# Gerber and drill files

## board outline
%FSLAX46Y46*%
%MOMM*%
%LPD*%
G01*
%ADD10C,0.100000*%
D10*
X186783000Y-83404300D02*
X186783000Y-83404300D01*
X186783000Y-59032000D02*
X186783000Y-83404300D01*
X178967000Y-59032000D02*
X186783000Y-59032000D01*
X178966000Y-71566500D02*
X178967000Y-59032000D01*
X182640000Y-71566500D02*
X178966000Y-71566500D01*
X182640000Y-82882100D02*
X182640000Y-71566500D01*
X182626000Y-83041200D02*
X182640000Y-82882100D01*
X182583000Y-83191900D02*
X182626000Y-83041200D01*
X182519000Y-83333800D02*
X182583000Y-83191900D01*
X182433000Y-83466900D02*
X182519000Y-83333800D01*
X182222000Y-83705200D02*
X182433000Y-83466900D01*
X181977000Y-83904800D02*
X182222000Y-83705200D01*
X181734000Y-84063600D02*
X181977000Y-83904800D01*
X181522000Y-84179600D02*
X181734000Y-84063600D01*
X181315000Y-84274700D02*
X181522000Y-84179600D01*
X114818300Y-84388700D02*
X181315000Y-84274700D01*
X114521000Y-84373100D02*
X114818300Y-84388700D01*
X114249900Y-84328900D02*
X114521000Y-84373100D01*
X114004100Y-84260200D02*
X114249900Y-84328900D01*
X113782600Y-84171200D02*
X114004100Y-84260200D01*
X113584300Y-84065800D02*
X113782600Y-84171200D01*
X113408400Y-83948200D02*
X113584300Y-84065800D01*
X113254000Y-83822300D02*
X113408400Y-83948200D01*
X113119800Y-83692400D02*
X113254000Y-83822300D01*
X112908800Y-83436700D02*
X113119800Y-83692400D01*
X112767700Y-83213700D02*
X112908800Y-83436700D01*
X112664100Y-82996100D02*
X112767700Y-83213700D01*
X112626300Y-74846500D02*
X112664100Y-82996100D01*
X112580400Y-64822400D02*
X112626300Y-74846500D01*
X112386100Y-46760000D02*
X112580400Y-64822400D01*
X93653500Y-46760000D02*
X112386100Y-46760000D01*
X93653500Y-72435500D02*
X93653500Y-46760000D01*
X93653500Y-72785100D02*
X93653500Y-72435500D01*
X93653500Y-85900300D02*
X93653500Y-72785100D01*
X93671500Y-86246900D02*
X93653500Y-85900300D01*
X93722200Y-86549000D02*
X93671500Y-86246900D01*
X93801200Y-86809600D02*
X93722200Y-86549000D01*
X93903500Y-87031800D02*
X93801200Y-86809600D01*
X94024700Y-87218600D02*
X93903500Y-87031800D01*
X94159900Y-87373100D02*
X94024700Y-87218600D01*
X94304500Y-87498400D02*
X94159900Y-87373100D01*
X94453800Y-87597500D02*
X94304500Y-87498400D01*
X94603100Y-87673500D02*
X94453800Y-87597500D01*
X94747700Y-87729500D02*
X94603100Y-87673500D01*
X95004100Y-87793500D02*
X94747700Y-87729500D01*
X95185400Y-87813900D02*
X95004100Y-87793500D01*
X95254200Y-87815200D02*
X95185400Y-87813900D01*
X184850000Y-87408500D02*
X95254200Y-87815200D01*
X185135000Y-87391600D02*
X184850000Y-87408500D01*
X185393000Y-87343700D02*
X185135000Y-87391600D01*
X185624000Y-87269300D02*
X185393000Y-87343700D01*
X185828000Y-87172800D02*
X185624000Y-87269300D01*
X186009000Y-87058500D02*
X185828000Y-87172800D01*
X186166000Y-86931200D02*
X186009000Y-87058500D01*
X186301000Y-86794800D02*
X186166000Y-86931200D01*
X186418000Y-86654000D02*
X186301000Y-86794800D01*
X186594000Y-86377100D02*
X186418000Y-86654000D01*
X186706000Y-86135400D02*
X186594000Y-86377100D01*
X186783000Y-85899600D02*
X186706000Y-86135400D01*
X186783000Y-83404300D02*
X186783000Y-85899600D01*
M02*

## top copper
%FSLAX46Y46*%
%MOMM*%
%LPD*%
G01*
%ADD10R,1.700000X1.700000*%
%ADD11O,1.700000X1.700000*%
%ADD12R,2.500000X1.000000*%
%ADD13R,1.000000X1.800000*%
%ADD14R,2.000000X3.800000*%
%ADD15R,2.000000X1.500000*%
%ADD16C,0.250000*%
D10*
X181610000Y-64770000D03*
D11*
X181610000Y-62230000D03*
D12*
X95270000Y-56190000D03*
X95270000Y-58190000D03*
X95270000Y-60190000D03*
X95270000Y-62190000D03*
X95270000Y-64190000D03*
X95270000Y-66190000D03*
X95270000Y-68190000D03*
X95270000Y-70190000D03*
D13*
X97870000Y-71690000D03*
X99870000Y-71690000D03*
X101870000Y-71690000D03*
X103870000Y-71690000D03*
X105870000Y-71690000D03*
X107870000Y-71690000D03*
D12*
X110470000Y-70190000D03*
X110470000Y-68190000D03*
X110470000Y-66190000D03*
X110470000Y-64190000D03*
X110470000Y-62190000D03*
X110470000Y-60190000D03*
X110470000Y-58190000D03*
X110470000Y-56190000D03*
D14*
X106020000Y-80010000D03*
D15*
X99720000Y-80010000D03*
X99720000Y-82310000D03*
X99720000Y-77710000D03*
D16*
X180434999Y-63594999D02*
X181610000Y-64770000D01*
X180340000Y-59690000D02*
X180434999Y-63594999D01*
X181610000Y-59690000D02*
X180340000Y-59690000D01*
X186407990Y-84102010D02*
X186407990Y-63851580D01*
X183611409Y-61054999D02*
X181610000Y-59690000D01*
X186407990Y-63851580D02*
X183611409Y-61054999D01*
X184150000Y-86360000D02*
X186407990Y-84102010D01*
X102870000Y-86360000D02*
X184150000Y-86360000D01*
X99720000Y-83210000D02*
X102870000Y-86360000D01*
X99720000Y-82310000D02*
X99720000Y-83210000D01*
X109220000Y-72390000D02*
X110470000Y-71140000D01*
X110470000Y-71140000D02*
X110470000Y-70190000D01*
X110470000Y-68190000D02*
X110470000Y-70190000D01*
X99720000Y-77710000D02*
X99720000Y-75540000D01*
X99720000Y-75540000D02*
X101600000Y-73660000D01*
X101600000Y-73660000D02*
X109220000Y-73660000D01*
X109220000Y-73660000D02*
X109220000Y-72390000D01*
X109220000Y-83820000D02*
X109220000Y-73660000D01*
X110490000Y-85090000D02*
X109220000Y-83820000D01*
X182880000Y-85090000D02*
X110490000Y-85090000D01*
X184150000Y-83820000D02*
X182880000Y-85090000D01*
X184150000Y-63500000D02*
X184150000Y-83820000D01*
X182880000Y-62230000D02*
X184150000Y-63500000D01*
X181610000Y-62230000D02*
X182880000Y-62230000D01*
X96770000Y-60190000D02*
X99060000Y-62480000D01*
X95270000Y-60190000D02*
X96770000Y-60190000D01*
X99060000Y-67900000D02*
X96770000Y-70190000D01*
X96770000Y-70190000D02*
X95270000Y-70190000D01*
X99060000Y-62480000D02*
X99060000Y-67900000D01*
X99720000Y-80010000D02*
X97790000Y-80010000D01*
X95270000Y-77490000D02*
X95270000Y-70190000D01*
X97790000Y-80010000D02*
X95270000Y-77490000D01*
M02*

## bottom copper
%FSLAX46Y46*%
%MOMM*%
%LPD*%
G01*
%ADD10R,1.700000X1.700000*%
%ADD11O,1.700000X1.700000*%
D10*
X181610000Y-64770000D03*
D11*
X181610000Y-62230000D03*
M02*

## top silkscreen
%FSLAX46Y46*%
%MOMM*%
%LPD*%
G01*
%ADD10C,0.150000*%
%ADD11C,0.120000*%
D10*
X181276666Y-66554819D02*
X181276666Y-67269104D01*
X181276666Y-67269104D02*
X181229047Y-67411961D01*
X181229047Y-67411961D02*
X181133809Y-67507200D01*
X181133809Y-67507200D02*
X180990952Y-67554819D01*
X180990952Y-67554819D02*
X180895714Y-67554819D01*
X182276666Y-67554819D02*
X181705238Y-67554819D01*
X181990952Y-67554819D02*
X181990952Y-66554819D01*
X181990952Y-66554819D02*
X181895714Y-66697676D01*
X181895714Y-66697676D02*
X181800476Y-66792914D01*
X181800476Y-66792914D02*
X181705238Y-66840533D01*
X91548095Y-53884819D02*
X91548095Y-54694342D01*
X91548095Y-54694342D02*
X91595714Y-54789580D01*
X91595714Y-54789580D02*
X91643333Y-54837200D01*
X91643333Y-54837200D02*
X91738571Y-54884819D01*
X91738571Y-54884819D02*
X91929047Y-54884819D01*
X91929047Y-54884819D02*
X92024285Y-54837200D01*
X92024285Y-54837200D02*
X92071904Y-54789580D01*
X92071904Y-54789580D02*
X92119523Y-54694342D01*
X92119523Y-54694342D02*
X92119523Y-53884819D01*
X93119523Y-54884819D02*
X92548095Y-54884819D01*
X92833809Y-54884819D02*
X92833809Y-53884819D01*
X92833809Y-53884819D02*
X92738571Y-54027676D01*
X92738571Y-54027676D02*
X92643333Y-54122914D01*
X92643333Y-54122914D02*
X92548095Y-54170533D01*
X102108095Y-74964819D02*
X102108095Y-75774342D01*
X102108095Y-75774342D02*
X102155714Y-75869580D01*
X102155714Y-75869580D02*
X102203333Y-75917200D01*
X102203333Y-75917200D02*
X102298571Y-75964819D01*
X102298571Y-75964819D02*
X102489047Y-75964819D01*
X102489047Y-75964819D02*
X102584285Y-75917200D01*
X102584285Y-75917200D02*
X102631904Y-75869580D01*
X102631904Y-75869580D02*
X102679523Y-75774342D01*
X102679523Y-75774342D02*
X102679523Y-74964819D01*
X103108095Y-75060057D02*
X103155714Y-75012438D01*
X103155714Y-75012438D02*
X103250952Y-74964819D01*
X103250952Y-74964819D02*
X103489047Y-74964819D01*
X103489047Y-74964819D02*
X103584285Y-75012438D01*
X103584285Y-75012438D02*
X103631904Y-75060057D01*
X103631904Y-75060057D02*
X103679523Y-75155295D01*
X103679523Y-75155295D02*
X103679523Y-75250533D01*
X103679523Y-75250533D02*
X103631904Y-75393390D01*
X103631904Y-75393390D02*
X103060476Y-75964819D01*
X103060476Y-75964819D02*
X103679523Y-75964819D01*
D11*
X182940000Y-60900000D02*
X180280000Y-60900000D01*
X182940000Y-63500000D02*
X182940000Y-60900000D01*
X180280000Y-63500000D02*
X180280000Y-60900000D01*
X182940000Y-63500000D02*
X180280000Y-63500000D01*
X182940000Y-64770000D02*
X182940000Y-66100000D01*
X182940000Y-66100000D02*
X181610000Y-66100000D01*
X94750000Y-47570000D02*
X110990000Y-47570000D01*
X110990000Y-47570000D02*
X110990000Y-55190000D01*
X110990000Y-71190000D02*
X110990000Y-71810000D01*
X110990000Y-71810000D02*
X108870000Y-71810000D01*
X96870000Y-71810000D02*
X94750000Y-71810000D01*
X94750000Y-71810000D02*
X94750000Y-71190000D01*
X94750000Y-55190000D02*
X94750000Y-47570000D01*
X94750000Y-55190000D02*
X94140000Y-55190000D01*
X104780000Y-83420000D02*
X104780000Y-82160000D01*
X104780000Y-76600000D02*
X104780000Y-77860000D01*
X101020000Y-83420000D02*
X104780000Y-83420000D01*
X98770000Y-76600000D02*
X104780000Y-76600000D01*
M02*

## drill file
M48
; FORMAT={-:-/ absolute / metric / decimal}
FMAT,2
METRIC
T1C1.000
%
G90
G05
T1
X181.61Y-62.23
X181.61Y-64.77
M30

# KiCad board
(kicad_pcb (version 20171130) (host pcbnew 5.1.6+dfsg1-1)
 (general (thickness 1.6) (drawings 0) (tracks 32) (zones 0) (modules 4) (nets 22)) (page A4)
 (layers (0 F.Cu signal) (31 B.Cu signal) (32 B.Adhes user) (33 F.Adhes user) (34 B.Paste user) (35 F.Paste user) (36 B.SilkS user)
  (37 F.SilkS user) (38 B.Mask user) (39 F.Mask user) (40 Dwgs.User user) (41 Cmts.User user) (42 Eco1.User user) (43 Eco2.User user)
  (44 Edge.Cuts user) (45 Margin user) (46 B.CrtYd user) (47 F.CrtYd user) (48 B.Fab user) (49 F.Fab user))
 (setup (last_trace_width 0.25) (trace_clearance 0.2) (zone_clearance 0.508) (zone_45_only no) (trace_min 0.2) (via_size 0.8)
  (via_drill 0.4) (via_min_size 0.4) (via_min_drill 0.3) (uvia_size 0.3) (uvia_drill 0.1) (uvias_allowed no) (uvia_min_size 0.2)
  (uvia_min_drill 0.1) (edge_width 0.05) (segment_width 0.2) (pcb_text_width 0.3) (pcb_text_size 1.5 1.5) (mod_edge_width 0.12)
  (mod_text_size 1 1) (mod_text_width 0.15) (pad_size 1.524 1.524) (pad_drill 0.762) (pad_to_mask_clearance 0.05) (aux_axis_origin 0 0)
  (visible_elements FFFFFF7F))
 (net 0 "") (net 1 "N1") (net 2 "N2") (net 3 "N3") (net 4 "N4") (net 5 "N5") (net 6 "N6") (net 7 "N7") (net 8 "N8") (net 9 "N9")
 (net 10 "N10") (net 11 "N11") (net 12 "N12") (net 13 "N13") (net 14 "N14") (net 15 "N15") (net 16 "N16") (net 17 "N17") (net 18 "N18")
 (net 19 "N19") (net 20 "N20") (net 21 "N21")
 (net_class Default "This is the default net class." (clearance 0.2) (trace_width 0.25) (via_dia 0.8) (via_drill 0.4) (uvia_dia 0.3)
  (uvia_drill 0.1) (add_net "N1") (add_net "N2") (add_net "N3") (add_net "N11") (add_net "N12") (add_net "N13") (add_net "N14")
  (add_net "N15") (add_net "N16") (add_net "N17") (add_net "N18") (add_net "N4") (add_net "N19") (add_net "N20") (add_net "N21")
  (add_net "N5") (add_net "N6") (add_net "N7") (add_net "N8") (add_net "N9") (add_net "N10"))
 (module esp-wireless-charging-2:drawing (layer F.Cu) (at 149.86 72.39)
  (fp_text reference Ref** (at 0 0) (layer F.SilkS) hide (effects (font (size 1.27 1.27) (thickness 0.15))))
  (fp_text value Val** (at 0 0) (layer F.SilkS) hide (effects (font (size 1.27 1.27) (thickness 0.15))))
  (fp_line (start 36.923 11.0143) (end 36.923 11.0143) (layer Edge.Cuts) (width 0.1))
  (fp_line (start 36.923 -13.358) (end 36.923 11.0143) (layer Edge.Cuts) (width 0.1))
  (fp_line (start 29.107 -13.358) (end 36.923 -13.358) (layer Edge.Cuts) (width 0.1))
  (fp_line (start 29.106 -0.8235) (end 29.107 -13.358) (layer Edge.Cuts) (width 0.1))
  (fp_line (start 32.78 -0.8235) (end 29.106 -0.8235) (layer Edge.Cuts) (width 0.1))
  (fp_line (start 32.78 10.4921) (end 32.78 -0.8235) (layer Edge.Cuts) (width 0.1))
  (fp_line (start 32.766 10.6512) (end 32.78 10.4921) (layer Edge.Cuts) (width 0.1))
  (fp_line (start 32.723 10.8019) (end 32.766 10.6512) (layer Edge.Cuts) (width 0.1))
  (fp_line (start 32.659 10.9438) (end 32.723 10.8019) (layer Edge.Cuts) (width 0.1))
  (fp_line (start 32.573 11.0769) (end 32.659 10.9438) (layer Edge.Cuts) (width 0.1))
  (fp_line (start 32.362 11.3152) (end 32.573 11.0769) (layer Edge.Cuts) (width 0.1))
  (fp_line (start 32.117 11.5148) (end 32.362 11.3152) (layer Edge.Cuts) (width 0.1))
  (fp_line (start 31.874 11.6736) (end 32.117 11.5148) (layer Edge.Cuts) (width 0.1))
  (fp_line (start 31.662 11.7896) (end 31.874 11.6736) (layer Edge.Cuts) (width 0.1))
  (fp_line (start 31.455 11.8847) (end 31.662 11.7896) (layer Edge.Cuts) (width 0.1))
  (fp_line (start -35.0417 11.9987) (end 31.455 11.8847) (layer Edge.Cuts) (width 0.1))
  (fp_line (start -35.339 11.9831) (end -35.0417 11.9987) (layer Edge.Cuts) (width 0.1))
  (fp_line (start -35.6101 11.9389) (end -35.339 11.9831) (layer Edge.Cuts) (width 0.1))
  (fp_line (start -35.8559 11.8702) (end -35.6101 11.9389) (layer Edge.Cuts) (width 0.1))
  (fp_line (start -36.0774 11.7812) (end -35.8559 11.8702) (layer Edge.Cuts) (width 0.1))
  (fp_line (start -36.2757 11.6758) (end -36.0774 11.7812) (layer Edge.Cuts) (width 0.1))
  (fp_line (start -36.4516 11.5582) (end -36.2757 11.6758) (layer Edge.Cuts) (width 0.1))
  (fp_line (start -36.606 11.4323) (end -36.4516 11.5582) (layer Edge.Cuts) (width 0.1))
  (fp_line (start -36.7402 11.3024) (end -36.606 11.4323) (layer Edge.Cuts) (width 0.1))
  (fp_line (start -36.9512 11.0467) (end -36.7402 11.3024) (layer Edge.Cuts) (width 0.1))
  (fp_line (start -37.0923 10.8237) (end -36.9512 11.0467) (layer Edge.Cuts) (width 0.1))
  (fp_line (start -37.1959 10.6061) (end -37.0923 10.8237) (layer Edge.Cuts) (width 0.1))
  (fp_line (start -37.2337 2.4565) (end -37.1959 10.6061) (layer Edge.Cuts) (width 0.1))
  (fp_line (start -37.2796 -7.5676) (end -37.2337 2.4565) (layer Edge.Cuts) (width 0.1))
  (fp_line (start -37.4739 -25.63) (end -37.2796 -7.5676) (layer Edge.Cuts) (width 0.1))
  (fp_line (start -56.2065 -25.63) (end -37.4739 -25.63) (layer Edge.Cuts) (width 0.1))
  (fp_line (start -56.2065 0.0455) (end -56.2065 -25.63) (layer Edge.Cuts) (width 0.1))
  (fp_line (start -56.2065 0.3951) (end -56.2065 0.0455) (layer Edge.Cuts) (width 0.1))
  (fp_line (start -56.2065 13.5103) (end -56.2065 0.3951) (layer Edge.Cuts) (width 0.1))
  (fp_line (start -56.1885 13.8569) (end -56.2065 13.5103) (layer Edge.Cuts) (width 0.1))
  (fp_line (start -56.1378 14.159) (end -56.1885 13.8569) (layer Edge.Cuts) (width 0.1))
  (fp_line (start -56.0588 14.4196) (end -56.1378 14.159) (layer Edge.Cuts) (width 0.1))
  (fp_line (start -55.9565 14.6418) (end -56.0588 14.4196) (layer Edge.Cuts) (width 0.1))
  (fp_line (start -55.8353 14.8286) (end -55.9565 14.6418) (layer Edge.Cuts) (width 0.1))
  (fp_line (start -55.7001 14.9831) (end -55.8353 14.8286) (layer Edge.Cuts) (width 0.1))
  (fp_line (start -55.5555 15.1084) (end -55.7001 14.9831) (layer Edge.Cuts) (width 0.1))
  (fp_line (start -55.4062 15.2075) (end -55.5555 15.1084) (layer Edge.Cuts) (width 0.1))
  (fp_line (start -55.2569 15.2835) (end -55.4062 15.2075) (layer Edge.Cuts) (width 0.1))
  (fp_line (start -55.1123 15.3395) (end -55.2569 15.2835) (layer Edge.Cuts) (width 0.1))
  (fp_line (start -54.8559 15.4035) (end -55.1123 15.3395) (layer Edge.Cuts) (width 0.1))
  (fp_line (start -54.6746 15.4239) (end -54.8559 15.4035) (layer Edge.Cuts) (width 0.1))
  (fp_line (start -54.6058 15.4252) (end -54.6746 15.4239) (layer Edge.Cuts) (width 0.1))
  (fp_line (start 34.99 15.0185) (end -54.6058 15.4252) (layer Edge.Cuts) (width 0.1))
  (fp_line (start 35.275 15.0016) (end 34.99 15.0185) (layer Edge.Cuts) (width 0.1))
  (fp_line (start 35.533 14.9537) (end 35.275 15.0016) (layer Edge.Cuts) (width 0.1))
  (fp_line (start 35.764 14.8793) (end 35.533 14.9537) (layer Edge.Cuts) (width 0.1))
  (fp_line (start 35.968 14.7828) (end 35.764 14.8793) (layer Edge.Cuts) (width 0.1))
  (fp_line (start 36.149 14.6685) (end 35.968 14.7828) (layer Edge.Cuts) (width 0.1))
  (fp_line (start 36.306 14.5412) (end 36.149 14.6685) (layer Edge.Cuts) (width 0.1))
  (fp_line (start 36.441 14.4048) (end 36.306 14.5412) (layer Edge.Cuts) (width 0.1))
  (fp_line (start 36.558 14.264) (end 36.441 14.4048) (layer Edge.Cuts) (width 0.1))
  (fp_line (start 36.734 13.9871) (end 36.558 14.264) (layer Edge.Cuts) (width 0.1))
  (fp_line (start 36.846 13.7454) (end 36.734 13.9871) (layer Edge.Cuts) (width 0.1))
  (fp_line (start 36.923 13.5096) (end 36.846 13.7454) (layer Edge.Cuts) (width 0.1))
  (fp_line (start 36.923 11.0143) (end 36.923 13.5096) (layer Edge.Cuts) (width 0.1)))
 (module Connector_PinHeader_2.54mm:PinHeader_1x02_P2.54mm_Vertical (layer F.Cu) (at 181.61 64.77 180)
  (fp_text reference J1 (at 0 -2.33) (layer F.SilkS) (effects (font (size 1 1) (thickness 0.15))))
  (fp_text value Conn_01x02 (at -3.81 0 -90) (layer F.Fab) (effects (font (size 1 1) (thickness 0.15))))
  (fp_line (start -1.33 3.87) (end 1.33 3.87) (layer F.SilkS) (width 0.12))
  (fp_line (start -1.33 1.27) (end -1.33 3.87) (layer F.SilkS) (width 0.12))
  (fp_line (start 1.33 1.27) (end 1.33 3.87) (layer F.SilkS) (width 0.12))
  (fp_line (start -1.33 1.27) (end 1.33 1.27) (layer F.SilkS) (width 0.12))
  (fp_line (start -1.33 0) (end -1.33 -1.33) (layer F.SilkS) (width 0.12))
  (fp_line (start -1.33 -1.33) (end 0 -1.33) (layer F.SilkS) (width 0.12))
  (pad 1 thru_hole rect (at 0 0 180) (size 1.7 1.7) (drill 1) (layers *.Cu *.Mask) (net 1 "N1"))
  (pad 2 thru_hole oval (at 0 2.54 180) (size 1.7 1.7) (drill 1) (layers *.Cu *.Mask) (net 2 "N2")))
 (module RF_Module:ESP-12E (layer F.Cu) (at 102.87 59.69)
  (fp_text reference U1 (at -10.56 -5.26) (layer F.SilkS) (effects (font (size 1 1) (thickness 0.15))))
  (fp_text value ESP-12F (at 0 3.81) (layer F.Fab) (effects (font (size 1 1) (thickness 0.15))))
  (fp_line (start -8.12 -12.12) (end 8.12 -12.12) (layer F.SilkS) (width 0.12))
  (fp_line (start 8.12 -12.12) (end 8.12 -4.5) (layer F.SilkS) (width 0.12))
  (fp_line (start 8.12 11.5) (end 8.12 12.12) (layer F.SilkS) (width 0.12))
  (fp_line (start 8.12 12.12) (end 6 12.12) (layer F.SilkS) (width 0.12))
  (fp_line (start -6 12.12) (end -8.12 12.12) (layer F.SilkS) (width 0.12))
  (fp_line (start -8.12 12.12) (end -8.12 11.5) (layer F.SilkS) (width 0.12))
  (fp_line (start -8.12 -4.5) (end -8.12 -12.12) (layer F.SilkS) (width 0.12))
  (fp_line (start -8.12 -4.5) (end -8.73 -4.5) (layer F.SilkS) (width 0.12))
  (pad 1 smd rect (at -7.6 -3.5) (size 2.5 1) (layers F.Cu F.Paste F.Mask) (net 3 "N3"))
  (pad 2 smd rect (at -7.6 -1.5) (size 2.5 1) (layers F.Cu F.Paste F.Mask) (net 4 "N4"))
  (pad 3 smd rect (at -7.6 0.5) (size 2.5 1) (layers F.Cu F.Paste F.Mask) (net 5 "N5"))
  (pad 4 smd rect (at -7.6 2.5) (size 2.5 1) (layers F.Cu F.Paste F.Mask) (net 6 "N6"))
  (pad 5 smd rect (at -7.6 4.5) (size 2.5 1) (layers F.Cu F.Paste F.Mask) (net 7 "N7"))
  (pad 6 smd rect (at -7.6 6.5) (size 2.5 1) (layers F.Cu F.Paste F.Mask) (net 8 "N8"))
  (pad 7 smd rect (at -7.6 8.5) (size 2.5 1) (layers F.Cu F.Paste F.Mask) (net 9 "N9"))
  (pad 8 smd rect (at -7.6 10.5) (size 2.5 1) (layers F.Cu F.Paste F.Mask) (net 5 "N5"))
  (pad 9 smd rect (at -5 12) (size 1 1.8) (layers F.Cu F.Paste F.Mask) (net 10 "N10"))
  (pad 10 smd rect (at -3 12) (size 1 1.8) (layers F.Cu F.Paste F.Mask) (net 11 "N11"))
  (pad 11 smd rect (at -1 12) (size 1 1.8) (layers F.Cu F.Paste F.Mask) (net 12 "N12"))
  (pad 12 smd rect (at 1 12) (size 1 1.8) (layers F.Cu F.Paste F.Mask) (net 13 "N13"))
  (pad 13 smd rect (at 3 12) (size 1 1.8) (layers F.Cu F.Paste F.Mask) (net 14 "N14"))
  (pad 14 smd rect (at 5 12) (size 1 1.8) (layers F.Cu F.Paste F.Mask) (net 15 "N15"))
  (pad 15 smd rect (at 7.6 10.5) (size 2.5 1) (layers F.Cu F.Paste F.Mask) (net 2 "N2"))
  (pad 16 smd rect (at 7.6 8.5) (size 2.5 1) (layers F.Cu F.Paste F.Mask) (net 2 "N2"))
  (pad 17 smd rect (at 7.6 6.5) (size 2.5 1) (layers F.Cu F.Paste F.Mask) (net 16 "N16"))
  (pad 18 smd rect (at 7.6 4.5) (size 2.5 1) (layers F.Cu F.Paste F.Mask) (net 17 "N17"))
  (pad 19 smd rect (at 7.6 2.5) (size 2.5 1) (layers F.Cu F.Paste F.Mask) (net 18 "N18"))
  (pad 20 smd rect (at 7.6 0.5) (size 2.5 1) (layers F.Cu F.Paste F.Mask) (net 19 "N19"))
  (pad 21 smd rect (at 7.6 -1.5) (size 2.5 1) (layers F.Cu F.Paste F.Mask) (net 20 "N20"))
  (pad 22 smd rect (at 7.6 -3.5) (size 2.5 1) (layers F.Cu F.Paste F.Mask) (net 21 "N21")))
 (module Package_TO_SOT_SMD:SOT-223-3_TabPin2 (layer F.Cu) (at 102.87 80.01)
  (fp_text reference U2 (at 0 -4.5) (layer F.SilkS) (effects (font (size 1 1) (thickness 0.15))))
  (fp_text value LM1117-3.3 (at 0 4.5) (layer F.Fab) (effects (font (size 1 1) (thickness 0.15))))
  (fp_line (start 1.91 3.41) (end 1.91 2.15) (layer F.SilkS) (width 0.12))
  (fp_line (start 1.91 -3.41) (end 1.91 -2.15) (layer F.SilkS) (width 0.12))
  (fp_line (start -1.85 3.41) (end 1.91 3.41) (layer F.SilkS) (width 0.12))
  (fp_line (start -4.1 -3.41) (end 1.91 -3.41) (layer F.SilkS) (width 0.12))
  (pad 2 smd rect (at 3.15 0) (size 2 3.8) (layers F.Cu F.Paste F.Mask) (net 5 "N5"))
  (pad 2 smd rect (at -3.15 0) (size 2 1.5) (layers F.Cu F.Paste F.Mask) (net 5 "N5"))
  (pad 3 smd rect (at -3.15 2.3) (size 2 1.5) (layers F.Cu F.Paste F.Mask) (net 1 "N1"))
  (pad 1 smd rect (at -3.15 -2.3) (size 2 1.5) (layers F.Cu F.Paste F.Mask) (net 2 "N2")))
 (segment (start 180.434999 63.594999) (end 181.61 64.77) (width 0.25) (layer F.Cu) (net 1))
 (segment (start 180.34 59.69) (end 180.434999 63.594999) (width 0.25) (layer F.Cu) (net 1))
 (segment (start 181.61 59.69) (end 180.34 59.69) (width 0.25) (layer F.Cu) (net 1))
 (segment (start 186.40799 84.10201) (end 186.40799 63.85158) (width 0.25) (layer F.Cu) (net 1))
 (segment (start 183.611409 61.054999) (end 181.61 59.69) (width 0.25) (layer F.Cu) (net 1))
 (segment (start 186.40799 63.85158) (end 183.611409 61.054999) (width 0.25) (layer F.Cu) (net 1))
 (segment (start 184.15 86.36) (end 186.40799 84.10201) (width 0.25) (layer F.Cu) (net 1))
 (segment (start 102.87 86.36) (end 184.15 86.36) (width 0.25) (layer F.Cu) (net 1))
 (segment (start 99.72 83.21) (end 102.87 86.36) (width 0.25) (layer F.Cu) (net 1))
 (segment (start 99.72 82.31) (end 99.72 83.21) (width 0.25) (layer F.Cu) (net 1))
 (segment (start 109.22 72.39) (end 110.47 71.14) (width 0.25) (layer F.Cu) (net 2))
 (segment (start 110.47 71.14) (end 110.47 70.19) (width 0.25) (layer F.Cu) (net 2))
 (segment (start 110.47 68.19) (end 110.47 70.19) (width 0.25) (layer F.Cu) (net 2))
 (segment (start 99.72 77.71) (end 99.72 75.54) (width 0.25) (layer F.Cu) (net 2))
 (segment (start 99.72 75.54) (end 101.6 73.66) (width 0.25) (layer F.Cu) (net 2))
 (segment (start 101.6 73.66) (end 109.22 73.66) (width 0.25) (layer F.Cu) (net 2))
 (segment (start 109.22 73.66) (end 109.22 72.39) (width 0.25) (layer F.Cu) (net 2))
 (segment (start 109.22 83.82) (end 109.22 73.66) (width 0.25) (layer F.Cu) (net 2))
 (segment (start 110.49 85.09) (end 109.22 83.82) (width 0.25) (layer F.Cu) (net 2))
 (segment (start 182.88 85.09) (end 110.49 85.09) (width 0.25) (layer F.Cu) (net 2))
 (segment (start 184.15 83.82) (end 182.88 85.09) (width 0.25) (layer F.Cu) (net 2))
 (segment (start 184.15 63.5) (end 184.15 83.82) (width 0.25) (layer F.Cu) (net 2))
 (segment (start 182.88 62.23) (end 184.15 63.5) (width 0.25) (layer F.Cu) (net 2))
 (segment (start 181.61 62.23) (end 182.88 62.23) (width 0.25) (layer F.Cu) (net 2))
 (segment (start 96.77 60.19) (end 99.06 62.48) (width 0.25) (layer F.Cu) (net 5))
 (segment (start 95.27 60.19) (end 96.77 60.19) (width 0.25) (layer F.Cu) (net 5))
 (segment (start 99.06 67.9) (end 96.77 70.19) (width 0.25) (layer F.Cu) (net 5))
 (segment (start 96.77 70.19) (end 95.27 70.19) (width 0.25) (layer F.Cu) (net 5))
 (segment (start 99.06 62.48) (end 99.06 67.9) (width 0.25) (layer F.Cu) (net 5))
 (segment (start 99.72 80.01) (end 97.79 80.01) (width 0.25) (layer F.Cu) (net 5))
 (segment (start 95.27 77.49) (end 95.27 70.19) (width 0.25) (layer F.Cu) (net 5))
 (segment (start 97.79 80.01) (end 95.27 77.49) (width 0.25) (layer F.Cu) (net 5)))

